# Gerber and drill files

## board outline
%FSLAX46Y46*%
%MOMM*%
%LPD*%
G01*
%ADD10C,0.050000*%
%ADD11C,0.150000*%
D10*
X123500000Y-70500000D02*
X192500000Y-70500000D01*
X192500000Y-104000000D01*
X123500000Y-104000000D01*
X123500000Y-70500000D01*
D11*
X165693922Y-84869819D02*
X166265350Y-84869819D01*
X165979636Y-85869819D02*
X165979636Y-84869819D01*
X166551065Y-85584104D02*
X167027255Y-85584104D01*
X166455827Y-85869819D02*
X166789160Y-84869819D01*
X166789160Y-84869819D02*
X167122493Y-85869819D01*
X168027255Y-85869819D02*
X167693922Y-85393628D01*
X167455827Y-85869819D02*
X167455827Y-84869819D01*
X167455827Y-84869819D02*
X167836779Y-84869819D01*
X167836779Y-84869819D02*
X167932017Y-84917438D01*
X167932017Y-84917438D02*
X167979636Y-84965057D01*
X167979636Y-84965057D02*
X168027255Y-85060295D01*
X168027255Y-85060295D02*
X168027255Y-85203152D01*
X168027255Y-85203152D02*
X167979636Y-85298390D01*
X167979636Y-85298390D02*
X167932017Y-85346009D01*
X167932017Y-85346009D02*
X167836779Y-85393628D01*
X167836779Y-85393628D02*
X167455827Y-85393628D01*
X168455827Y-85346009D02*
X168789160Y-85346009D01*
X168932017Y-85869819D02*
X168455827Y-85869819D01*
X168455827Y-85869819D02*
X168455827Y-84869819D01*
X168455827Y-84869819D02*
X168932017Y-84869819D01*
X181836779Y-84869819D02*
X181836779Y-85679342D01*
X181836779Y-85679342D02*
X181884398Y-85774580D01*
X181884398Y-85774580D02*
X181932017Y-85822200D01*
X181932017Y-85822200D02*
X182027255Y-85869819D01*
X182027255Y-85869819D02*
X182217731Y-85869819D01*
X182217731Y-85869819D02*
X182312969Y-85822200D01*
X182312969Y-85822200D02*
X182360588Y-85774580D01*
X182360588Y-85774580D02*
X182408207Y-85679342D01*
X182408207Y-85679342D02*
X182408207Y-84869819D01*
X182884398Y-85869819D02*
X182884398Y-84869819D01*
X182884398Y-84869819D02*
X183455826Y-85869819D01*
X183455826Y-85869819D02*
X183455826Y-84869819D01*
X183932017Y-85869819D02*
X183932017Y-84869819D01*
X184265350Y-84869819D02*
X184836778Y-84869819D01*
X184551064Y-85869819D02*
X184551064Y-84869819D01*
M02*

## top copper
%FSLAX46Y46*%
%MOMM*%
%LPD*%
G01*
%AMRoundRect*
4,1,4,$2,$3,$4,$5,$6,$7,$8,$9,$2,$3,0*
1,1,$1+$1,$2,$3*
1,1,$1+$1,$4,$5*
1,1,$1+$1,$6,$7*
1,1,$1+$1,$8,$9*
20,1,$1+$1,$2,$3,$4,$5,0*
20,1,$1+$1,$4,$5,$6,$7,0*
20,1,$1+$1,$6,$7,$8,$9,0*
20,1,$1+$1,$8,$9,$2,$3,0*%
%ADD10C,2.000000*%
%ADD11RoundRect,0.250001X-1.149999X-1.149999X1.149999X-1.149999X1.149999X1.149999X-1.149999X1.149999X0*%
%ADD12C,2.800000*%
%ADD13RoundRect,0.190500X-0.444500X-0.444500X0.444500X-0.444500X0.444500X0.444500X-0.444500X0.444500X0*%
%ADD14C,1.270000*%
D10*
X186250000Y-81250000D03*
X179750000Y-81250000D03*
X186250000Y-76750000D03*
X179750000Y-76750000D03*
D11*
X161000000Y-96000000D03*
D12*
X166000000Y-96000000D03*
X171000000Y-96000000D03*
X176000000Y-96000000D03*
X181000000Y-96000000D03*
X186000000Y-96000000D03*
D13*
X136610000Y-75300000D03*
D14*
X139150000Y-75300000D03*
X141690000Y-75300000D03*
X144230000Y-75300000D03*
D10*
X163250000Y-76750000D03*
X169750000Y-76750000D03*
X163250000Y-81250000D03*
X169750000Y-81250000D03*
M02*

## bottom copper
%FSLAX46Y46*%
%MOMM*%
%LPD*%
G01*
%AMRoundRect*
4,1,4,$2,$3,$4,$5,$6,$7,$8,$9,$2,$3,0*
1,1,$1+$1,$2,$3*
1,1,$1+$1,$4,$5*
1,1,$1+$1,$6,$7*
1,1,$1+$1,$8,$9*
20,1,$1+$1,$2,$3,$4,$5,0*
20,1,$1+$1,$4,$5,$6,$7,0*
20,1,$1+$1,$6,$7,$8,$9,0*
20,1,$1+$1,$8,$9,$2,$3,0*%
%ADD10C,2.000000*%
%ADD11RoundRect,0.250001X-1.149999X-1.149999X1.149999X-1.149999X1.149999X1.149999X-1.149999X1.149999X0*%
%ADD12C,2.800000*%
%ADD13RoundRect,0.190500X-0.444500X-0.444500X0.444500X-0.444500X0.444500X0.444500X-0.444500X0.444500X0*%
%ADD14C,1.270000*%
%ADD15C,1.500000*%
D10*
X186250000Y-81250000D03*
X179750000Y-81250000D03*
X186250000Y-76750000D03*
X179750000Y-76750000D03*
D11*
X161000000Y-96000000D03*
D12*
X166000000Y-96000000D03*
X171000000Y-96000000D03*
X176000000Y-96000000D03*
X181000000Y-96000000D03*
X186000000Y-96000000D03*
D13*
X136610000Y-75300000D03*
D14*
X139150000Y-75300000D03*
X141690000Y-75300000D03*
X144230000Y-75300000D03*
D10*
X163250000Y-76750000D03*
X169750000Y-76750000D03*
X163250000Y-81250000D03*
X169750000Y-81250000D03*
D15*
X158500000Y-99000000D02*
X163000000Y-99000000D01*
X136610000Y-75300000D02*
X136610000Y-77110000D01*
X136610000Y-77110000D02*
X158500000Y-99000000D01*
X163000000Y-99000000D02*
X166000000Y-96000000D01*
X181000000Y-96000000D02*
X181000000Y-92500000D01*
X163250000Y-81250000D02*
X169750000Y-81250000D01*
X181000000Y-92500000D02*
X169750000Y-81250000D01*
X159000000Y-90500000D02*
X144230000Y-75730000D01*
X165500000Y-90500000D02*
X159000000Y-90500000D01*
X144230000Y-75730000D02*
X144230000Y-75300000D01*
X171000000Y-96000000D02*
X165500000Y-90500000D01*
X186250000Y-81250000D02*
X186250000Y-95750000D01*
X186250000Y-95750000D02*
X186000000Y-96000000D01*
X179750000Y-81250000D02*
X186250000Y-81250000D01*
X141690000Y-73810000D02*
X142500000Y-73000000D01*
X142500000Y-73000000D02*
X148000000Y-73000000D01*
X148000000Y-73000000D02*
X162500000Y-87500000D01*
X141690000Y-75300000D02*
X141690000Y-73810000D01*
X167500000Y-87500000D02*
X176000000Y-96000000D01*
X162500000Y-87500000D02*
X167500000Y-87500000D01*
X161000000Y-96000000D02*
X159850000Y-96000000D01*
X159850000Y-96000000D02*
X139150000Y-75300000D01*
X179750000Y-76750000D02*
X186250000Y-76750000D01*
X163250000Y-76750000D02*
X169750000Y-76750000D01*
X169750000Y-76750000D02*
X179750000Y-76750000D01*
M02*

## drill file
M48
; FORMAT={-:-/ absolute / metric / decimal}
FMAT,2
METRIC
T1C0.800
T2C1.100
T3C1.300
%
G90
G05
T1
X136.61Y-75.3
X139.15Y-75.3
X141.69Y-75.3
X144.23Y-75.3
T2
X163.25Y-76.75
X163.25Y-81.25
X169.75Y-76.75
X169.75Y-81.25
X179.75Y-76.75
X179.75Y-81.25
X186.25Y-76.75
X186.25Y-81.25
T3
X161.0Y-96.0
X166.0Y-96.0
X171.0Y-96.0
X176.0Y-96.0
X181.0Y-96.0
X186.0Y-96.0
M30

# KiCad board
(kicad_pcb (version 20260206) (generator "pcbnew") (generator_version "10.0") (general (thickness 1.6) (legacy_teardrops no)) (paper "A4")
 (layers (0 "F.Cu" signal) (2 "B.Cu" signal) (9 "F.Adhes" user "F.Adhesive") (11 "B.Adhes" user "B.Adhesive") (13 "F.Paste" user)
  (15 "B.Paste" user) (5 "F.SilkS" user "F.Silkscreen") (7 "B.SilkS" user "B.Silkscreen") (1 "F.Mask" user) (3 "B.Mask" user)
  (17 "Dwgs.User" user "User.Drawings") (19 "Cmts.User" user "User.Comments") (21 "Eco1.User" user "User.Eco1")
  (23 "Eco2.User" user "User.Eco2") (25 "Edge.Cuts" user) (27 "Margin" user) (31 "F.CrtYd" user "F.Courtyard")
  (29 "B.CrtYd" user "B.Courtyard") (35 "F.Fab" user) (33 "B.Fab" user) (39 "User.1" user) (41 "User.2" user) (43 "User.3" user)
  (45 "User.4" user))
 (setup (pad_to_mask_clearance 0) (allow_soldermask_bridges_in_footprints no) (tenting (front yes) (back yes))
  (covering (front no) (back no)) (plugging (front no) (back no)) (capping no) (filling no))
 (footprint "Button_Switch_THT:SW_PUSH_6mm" (layer "F.Cu") (at 186.25 81.25 180)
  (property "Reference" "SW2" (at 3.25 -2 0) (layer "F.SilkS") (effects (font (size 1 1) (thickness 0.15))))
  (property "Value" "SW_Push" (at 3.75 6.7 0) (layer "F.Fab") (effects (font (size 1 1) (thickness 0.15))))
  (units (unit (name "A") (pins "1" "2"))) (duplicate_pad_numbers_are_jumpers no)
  (pad "1" thru_hole circle (at 0 0 270) (size 2 2) (drill 1.1) (layers "*.Cu" "*.Mask") (remove_unused_layers no) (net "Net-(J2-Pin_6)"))
  (pad "1" thru_hole circle (at 6.5 0 270) (size 2 2) (drill 1.1) (layers "*.Cu" "*.Mask") (remove_unused_layers no) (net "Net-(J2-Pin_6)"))
  (pad "2" thru_hole circle (at 0 4.5 270) (size 2 2) (drill 1.1) (layers "*.Cu" "*.Mask") (remove_unused_layers no) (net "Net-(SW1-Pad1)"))
  (pad "2" thru_hole circle (at 6.5 4.5 270) (size 2 2) (drill 1.1) (layers "*.Cu" "*.Mask") (remove_unused_layers no)
   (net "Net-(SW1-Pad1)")))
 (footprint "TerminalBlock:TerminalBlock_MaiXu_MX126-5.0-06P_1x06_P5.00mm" (layer "F.Cu") (at 161 96)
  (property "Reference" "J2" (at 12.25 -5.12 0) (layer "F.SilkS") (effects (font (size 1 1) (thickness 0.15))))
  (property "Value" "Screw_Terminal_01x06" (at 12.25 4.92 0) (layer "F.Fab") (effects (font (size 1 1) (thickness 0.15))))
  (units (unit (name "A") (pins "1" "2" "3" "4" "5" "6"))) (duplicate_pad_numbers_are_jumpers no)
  (pad "1" thru_hole roundrect (at 0 0) (size 2.8 2.8) (drill 1.3) (layers "*.Cu" "*.Mask") (remove_unused_layers no)
   (roundrect_rratio 0.089286) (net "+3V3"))
  (pad "2" thru_hole circle (at 5 0) (size 2.8 2.8) (drill 1.3) (layers "*.Cu" "*.Mask") (remove_unused_layers no) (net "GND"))
  (pad "3" thru_hole circle (at 10 0) (size 2.8 2.8) (drill 1.3) (layers "*.Cu" "*.Mask") (remove_unused_layers no) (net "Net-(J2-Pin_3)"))
  (pad "4" thru_hole circle (at 15 0) (size 2.8 2.8) (drill 1.3) (layers "*.Cu" "*.Mask") (remove_unused_layers no) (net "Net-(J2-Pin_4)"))
  (pad "5" thru_hole circle (at 20 0) (size 2.8 2.8) (drill 1.3) (layers "*.Cu" "*.Mask") (remove_unused_layers no) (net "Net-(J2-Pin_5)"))
  (pad "6" thru_hole circle (at 25 0) (size 2.8 2.8) (drill 1.3) (layers "*.Cu" "*.Mask") (remove_unused_layers no) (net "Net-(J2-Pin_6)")))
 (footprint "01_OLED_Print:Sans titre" (layer "F.Cu") (at 140.5 88)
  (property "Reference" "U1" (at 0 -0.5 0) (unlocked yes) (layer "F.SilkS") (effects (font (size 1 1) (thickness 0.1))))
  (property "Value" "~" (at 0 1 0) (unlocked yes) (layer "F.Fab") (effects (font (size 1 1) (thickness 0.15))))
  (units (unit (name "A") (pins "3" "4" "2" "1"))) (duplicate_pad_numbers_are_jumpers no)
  (pad "1" thru_hole roundrect (at -3.89 -12.7) (size 1.27 1.27) (drill 0.8) (layers "*.Cu" "*.Mask") (remove_unused_layers no)
   (roundrect_rratio 0.15) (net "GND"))
  (pad "2" thru_hole circle (at -1.35 -12.7) (size 1.27 1.27) (drill 0.8) (layers "*.Cu" "*.Mask") (remove_unused_layers no) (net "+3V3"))
  (pad "3" thru_hole circle (at 1.19 -12.7) (size 1.27 1.27) (drill 0.8) (layers "*.Cu" "*.Mask") (remove_unused_layers no)
   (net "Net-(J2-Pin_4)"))
  (pad "4" thru_hole circle (at 3.73 -12.7) (size 1.27 1.27) (drill 0.8) (layers "*.Cu" "*.Mask") (remove_unused_layers no)
   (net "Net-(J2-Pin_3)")))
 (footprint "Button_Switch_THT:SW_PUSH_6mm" (layer "F.Cu") (at 163.25 76.75)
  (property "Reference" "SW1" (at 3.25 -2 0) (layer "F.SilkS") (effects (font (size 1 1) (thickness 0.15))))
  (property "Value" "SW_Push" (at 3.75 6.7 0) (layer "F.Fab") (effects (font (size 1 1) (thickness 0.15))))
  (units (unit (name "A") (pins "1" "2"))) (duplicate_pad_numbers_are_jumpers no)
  (pad "1" thru_hole circle (at 0 0 90) (size 2 2) (drill 1.1) (layers "*.Cu" "*.Mask") (remove_unused_layers no) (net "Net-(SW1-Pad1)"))
  (pad "1" thru_hole circle (at 6.5 0 90) (size 2 2) (drill 1.1) (layers "*.Cu" "*.Mask") (remove_unused_layers no) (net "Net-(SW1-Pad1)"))
  (pad "2" thru_hole circle (at 0 4.5 90) (size 2 2) (drill 1.1) (layers "*.Cu" "*.Mask") (remove_unused_layers no) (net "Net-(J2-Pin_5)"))
  (pad "2" thru_hole circle (at 6.5 4.5 90) (size 2 2) (drill 1.1) (layers "*.Cu" "*.Mask") (remove_unused_layers no) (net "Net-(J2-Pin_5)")))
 (gr_rect (start 123.5 70.5) (end 192.5 104) (stroke (width 0.05) (type default)) (fill no) (layer "Edge.Cuts"))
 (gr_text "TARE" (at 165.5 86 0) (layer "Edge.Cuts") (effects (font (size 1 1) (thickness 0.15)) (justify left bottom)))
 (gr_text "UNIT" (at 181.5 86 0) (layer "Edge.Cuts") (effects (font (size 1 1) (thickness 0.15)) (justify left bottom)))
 (segment (start 158.5 99) (end 163 99) (width 1.5) (layer "B.Cu") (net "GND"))
 (segment (start 136.61 75.3) (end 136.61 77.11) (width 1.5) (layer "B.Cu") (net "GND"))
 (segment (start 136.61 77.11) (end 158.5 99) (width 1.5) (layer "B.Cu") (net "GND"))
 (segment (start 163 99) (end 166 96) (width 1.5) (layer "B.Cu") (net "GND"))
 (segment (start 181 96) (end 181 92.5) (width 1.5) (layer "B.Cu") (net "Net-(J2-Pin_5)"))
 (segment (start 163.25 81.25) (end 169.75 81.25) (width 1.5) (layer "B.Cu") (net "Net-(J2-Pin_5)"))
 (segment (start 181 92.5) (end 169.75 81.25) (width 1.5) (layer "B.Cu") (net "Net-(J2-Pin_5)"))
 (segment (start 159 90.5) (end 144.23 75.73) (width 1.5) (layer "B.Cu") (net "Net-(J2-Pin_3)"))
 (segment (start 165.5 90.5) (end 159 90.5) (width 1.5) (layer "B.Cu") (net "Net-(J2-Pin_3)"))
 (segment (start 144.23 75.73) (end 144.23 75.3) (width 1.5) (layer "B.Cu") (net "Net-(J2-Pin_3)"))
 (segment (start 171 96) (end 165.5 90.5) (width 1.5) (layer "B.Cu") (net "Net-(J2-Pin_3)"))
 (segment (start 186.25 81.25) (end 186.25 95.75) (width 1.5) (layer "B.Cu") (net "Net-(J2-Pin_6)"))
 (segment (start 186.25 95.75) (end 186 96) (width 1.5) (layer "B.Cu") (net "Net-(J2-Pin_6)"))
 (segment (start 179.75 81.25) (end 186.25 81.25) (width 1.5) (layer "B.Cu") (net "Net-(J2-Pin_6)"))
 (segment (start 141.69 73.81) (end 142.5 73) (width 1.5) (layer "B.Cu") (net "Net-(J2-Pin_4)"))
 (segment (start 142.5 73) (end 148 73) (width 1.5) (layer "B.Cu") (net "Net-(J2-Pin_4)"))
 (segment (start 148 73) (end 162.5 87.5) (width 1.5) (layer "B.Cu") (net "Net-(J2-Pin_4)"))
 (segment (start 141.69 75.3) (end 141.69 73.81) (width 1.5) (layer "B.Cu") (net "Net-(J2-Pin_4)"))
 (segment (start 167.5 87.5) (end 176 96) (width 1.5) (layer "B.Cu") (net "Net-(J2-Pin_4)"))
 (segment (start 162.5 87.5) (end 167.5 87.5) (width 1.5) (layer "B.Cu") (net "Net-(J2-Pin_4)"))
 (segment (start 161 96) (end 159.85 96) (width 1.5) (layer "B.Cu") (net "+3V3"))
 (segment (start 159.85 96) (end 139.15 75.3) (width 1.5) (layer "B.Cu") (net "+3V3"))
 (segment (start 179.75 76.75) (end 186.25 76.75) (width 1.5) (layer "B.Cu") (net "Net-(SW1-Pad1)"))
 (segment (start 163.25 76.75) (end 169.75 76.75) (width 1.5) (layer "B.Cu") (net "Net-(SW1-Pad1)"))
 (segment (start 169.75 76.75) (end 179.75 76.75) (width 1.5) (layer "B.Cu") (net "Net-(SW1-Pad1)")))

